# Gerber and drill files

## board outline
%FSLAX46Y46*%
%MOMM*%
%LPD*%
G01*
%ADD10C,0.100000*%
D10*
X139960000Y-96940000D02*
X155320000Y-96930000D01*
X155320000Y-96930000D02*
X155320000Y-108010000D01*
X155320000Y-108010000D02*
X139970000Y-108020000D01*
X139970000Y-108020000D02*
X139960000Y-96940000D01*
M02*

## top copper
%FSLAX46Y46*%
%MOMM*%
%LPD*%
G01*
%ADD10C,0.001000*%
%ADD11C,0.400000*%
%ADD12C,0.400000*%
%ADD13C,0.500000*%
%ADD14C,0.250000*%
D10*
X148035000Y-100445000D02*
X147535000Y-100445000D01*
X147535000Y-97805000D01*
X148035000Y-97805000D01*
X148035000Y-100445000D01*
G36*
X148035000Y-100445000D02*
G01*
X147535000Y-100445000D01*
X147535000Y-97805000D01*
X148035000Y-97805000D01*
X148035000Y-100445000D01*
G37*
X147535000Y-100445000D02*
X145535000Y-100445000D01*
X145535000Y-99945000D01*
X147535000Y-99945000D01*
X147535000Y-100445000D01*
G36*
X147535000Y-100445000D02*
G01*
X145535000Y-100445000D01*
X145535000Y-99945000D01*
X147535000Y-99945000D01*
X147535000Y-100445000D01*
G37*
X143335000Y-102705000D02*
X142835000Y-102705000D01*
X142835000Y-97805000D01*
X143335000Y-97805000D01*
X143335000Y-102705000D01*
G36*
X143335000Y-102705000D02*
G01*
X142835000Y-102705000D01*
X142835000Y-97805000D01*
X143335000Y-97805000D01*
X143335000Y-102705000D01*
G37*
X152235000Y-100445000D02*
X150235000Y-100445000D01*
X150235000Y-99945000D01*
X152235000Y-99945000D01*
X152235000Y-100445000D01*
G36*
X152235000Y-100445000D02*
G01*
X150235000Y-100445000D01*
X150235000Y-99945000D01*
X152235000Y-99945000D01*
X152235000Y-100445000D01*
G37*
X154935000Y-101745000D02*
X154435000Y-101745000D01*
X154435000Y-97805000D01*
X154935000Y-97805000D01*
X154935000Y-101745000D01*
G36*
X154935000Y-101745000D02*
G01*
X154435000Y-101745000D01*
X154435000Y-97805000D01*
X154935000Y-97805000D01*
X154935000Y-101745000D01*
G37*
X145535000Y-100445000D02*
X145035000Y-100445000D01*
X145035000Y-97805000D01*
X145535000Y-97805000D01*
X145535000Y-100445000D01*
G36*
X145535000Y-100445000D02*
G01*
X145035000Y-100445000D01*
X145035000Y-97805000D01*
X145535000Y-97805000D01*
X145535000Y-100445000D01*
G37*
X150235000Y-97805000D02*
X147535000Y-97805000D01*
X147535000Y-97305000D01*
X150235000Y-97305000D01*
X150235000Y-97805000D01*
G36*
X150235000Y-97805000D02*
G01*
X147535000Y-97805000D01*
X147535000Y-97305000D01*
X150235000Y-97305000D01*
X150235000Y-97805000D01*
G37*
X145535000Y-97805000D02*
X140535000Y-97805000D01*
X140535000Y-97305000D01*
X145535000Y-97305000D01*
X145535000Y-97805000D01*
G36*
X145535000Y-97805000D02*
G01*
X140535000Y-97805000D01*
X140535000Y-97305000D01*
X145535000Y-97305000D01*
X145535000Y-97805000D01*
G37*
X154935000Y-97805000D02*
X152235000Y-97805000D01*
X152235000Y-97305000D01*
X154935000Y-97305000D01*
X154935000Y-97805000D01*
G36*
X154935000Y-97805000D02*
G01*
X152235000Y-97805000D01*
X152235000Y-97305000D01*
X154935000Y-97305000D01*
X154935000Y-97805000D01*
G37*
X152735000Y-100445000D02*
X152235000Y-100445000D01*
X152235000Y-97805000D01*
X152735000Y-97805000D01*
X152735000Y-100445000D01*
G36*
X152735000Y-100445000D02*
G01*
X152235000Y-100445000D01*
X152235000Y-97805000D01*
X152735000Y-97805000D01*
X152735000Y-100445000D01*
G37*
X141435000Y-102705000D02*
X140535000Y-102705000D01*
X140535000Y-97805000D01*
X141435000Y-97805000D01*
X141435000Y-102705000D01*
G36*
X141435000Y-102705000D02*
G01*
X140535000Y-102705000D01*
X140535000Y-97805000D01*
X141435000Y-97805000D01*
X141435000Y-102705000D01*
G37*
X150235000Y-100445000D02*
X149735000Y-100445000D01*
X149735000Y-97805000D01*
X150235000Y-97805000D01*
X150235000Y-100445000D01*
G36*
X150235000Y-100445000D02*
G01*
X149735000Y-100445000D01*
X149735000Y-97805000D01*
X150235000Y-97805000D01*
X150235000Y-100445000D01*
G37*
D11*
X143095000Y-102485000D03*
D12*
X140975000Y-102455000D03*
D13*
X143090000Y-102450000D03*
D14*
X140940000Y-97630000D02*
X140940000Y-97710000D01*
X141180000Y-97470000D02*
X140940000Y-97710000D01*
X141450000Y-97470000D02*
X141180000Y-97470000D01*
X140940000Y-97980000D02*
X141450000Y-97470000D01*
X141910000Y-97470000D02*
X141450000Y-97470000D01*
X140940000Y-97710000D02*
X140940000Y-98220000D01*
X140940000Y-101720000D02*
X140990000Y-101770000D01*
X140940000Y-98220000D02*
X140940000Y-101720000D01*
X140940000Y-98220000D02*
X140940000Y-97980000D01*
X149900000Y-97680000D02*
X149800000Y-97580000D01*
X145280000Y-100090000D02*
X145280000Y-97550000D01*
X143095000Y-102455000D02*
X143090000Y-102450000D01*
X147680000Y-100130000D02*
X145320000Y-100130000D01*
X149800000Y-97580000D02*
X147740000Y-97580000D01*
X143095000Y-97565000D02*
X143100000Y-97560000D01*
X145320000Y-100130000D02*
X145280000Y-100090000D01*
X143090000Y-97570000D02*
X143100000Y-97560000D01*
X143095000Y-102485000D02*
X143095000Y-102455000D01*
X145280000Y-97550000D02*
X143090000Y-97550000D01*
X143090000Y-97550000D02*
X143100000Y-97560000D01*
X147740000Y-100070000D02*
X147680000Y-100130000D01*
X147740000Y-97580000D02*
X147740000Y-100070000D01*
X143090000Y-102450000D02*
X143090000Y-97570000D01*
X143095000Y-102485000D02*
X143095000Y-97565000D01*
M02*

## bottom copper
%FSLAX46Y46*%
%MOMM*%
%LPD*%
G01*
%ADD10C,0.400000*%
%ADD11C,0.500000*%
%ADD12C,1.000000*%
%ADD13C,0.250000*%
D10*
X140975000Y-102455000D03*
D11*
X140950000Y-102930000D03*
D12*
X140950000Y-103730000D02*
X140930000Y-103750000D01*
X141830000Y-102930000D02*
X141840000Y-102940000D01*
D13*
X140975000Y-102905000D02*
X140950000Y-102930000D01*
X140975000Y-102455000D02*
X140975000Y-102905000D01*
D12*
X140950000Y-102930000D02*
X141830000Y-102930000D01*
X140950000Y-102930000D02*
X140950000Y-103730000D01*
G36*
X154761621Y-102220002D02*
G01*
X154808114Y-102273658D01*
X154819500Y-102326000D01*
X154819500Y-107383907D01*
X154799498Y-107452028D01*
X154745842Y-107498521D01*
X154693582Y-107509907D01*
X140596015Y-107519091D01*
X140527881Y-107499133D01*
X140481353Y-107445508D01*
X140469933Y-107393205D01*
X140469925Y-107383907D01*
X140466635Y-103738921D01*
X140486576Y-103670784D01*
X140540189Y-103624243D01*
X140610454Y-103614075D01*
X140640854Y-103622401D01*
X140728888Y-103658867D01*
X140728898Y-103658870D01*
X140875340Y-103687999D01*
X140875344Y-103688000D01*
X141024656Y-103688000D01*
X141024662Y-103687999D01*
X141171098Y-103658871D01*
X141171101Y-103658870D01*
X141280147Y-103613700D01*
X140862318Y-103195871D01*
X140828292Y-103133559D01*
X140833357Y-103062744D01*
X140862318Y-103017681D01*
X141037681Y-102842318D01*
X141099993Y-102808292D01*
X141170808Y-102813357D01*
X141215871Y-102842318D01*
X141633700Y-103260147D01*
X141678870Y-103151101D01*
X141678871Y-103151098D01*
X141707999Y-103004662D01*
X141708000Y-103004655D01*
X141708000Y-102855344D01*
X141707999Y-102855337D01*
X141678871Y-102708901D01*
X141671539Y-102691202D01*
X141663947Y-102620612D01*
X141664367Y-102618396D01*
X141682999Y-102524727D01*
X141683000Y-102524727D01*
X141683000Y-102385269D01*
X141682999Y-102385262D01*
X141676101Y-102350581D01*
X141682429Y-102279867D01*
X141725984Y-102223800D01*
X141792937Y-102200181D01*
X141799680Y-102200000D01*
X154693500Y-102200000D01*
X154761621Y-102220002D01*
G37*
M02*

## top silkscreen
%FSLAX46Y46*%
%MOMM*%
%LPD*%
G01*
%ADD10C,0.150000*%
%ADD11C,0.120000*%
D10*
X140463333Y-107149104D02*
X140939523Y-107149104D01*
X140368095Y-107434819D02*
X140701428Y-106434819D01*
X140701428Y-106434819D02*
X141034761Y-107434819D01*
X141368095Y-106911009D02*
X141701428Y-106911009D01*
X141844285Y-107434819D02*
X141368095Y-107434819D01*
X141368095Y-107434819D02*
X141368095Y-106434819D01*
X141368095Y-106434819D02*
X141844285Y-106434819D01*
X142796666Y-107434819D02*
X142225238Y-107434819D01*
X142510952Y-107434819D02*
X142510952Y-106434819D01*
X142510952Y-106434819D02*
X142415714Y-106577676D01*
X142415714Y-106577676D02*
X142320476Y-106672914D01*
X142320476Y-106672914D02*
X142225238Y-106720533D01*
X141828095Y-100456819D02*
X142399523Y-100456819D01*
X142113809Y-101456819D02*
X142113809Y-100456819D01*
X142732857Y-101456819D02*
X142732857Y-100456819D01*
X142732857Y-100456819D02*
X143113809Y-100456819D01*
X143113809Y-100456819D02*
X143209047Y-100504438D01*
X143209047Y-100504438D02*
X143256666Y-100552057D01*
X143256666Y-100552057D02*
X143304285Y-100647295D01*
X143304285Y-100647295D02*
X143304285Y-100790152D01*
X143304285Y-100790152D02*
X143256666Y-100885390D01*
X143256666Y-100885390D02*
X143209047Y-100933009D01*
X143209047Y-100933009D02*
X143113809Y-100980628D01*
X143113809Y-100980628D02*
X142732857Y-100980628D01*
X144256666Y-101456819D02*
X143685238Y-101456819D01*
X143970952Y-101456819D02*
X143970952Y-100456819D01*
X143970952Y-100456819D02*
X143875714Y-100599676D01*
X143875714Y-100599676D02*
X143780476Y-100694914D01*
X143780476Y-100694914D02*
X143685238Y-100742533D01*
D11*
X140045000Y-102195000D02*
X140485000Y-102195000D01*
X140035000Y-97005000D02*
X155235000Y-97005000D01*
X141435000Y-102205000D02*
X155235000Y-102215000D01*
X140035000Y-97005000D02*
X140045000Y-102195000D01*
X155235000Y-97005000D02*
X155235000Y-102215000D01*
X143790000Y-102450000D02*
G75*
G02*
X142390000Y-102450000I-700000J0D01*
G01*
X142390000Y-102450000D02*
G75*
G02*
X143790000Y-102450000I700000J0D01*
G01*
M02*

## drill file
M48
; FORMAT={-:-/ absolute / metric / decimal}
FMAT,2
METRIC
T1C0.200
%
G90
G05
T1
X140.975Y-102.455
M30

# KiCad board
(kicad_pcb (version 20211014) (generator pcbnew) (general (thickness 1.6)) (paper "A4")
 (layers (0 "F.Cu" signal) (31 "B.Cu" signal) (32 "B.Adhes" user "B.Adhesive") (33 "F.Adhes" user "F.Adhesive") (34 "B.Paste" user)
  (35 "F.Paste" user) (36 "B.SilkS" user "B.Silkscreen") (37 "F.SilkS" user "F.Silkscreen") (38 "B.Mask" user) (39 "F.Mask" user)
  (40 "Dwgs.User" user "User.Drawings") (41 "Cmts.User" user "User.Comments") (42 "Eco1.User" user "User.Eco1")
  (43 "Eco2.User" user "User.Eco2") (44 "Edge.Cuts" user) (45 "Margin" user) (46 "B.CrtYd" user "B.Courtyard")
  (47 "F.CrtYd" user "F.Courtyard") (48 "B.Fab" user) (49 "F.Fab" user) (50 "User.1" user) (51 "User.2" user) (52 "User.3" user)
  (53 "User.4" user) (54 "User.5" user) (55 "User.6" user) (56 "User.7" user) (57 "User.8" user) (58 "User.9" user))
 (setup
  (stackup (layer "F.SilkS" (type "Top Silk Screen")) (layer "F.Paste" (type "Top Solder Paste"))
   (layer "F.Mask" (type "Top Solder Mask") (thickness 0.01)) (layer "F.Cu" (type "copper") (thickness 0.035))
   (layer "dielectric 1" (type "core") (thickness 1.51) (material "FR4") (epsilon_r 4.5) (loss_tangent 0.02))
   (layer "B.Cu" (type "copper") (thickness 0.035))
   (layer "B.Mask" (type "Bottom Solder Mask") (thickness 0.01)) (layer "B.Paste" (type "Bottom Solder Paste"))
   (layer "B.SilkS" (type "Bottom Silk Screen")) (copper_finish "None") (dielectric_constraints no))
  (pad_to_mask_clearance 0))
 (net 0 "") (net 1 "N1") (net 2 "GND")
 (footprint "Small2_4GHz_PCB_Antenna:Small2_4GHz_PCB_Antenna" (layer "F.Cu") (at 140.535 97.305)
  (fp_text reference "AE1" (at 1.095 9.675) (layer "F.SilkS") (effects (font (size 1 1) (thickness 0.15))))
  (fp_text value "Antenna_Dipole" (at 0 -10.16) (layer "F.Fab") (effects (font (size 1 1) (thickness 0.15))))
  (fp_poly (pts (xy 7.5 3.14) (xy 7 3.14) (xy 7 0.5) (xy 7.5 0.5)) (layer "F.Cu") (width 0.001) (fill solid))
  (fp_poly (pts (xy 7 3.14) (xy 5 3.14) (xy 5 2.64) (xy 7 2.64)) (layer "F.Cu") (width 0.001) (fill solid))
  (fp_poly (pts (xy 2.8 5.4) (xy 2.3 5.4) (xy 2.3 0.5) (xy 2.8 0.5)) (layer "F.Cu") (width 0.001) (fill solid))
  (fp_poly (pts (xy 11.7 3.14) (xy 9.7 3.14) (xy 9.7 2.64) (xy 11.7 2.64)) (layer "F.Cu") (width 0.001) (fill solid))
  (fp_poly (pts (xy 14.4 4.44) (xy 13.9 4.44) (xy 13.9 0.5) (xy 14.4 0.5)) (layer "F.Cu") (width 0.001) (fill solid))
  (fp_poly (pts (xy 5 3.14) (xy 4.5 3.14) (xy 4.5 0.5) (xy 5 0.5)) (layer "F.Cu") (width 0.001) (fill solid))
  (fp_poly (pts (xy 9.7 0.5) (xy 7 0.5) (xy 7 0) (xy 9.7 0)) (layer "F.Cu") (width 0.001) (fill solid))
  (fp_poly (pts (xy 5 0.5) (xy 0 0.5) (xy 0 0) (xy 5 0)) (layer "F.Cu") (width 0.001) (fill solid))
  (fp_poly (pts (xy 14.4 0.5) (xy 11.7 0.5) (xy 11.7 0) (xy 14.4 0)) (layer "F.Cu") (width 0.001) (fill solid))
  (fp_poly (pts (xy 12.2 3.14) (xy 11.7 3.14) (xy 11.7 0.5) (xy 12.2 0.5)) (layer "F.Cu") (width 0.001) (fill solid))
  (fp_poly (pts (xy 0.9 5.4) (xy 0 5.4) (xy 0 0.5) (xy 0.9 0.5)) (layer "F.Cu") (width 0.001) (fill solid))
  (fp_poly (pts (xy 9.7 3.14) (xy 9.2 3.14) (xy 9.2 0.5) (xy 9.7 0.5)) (layer "F.Cu") (width 0.001) (fill solid))
  (fp_line (start -0.49 4.89) (end -0.05 4.89) (layer "F.SilkS") (width 0.12))
  (fp_line (start -0.5 -0.3) (end 14.7 -0.3) (layer "F.SilkS") (width 0.12))
  (fp_line (start 0.9 4.9) (end 14.7 4.91) (layer "F.SilkS") (width 0.12))
  (fp_line (start -0.5 -0.3) (end -0.49 4.89) (layer "F.SilkS") (width 0.12))
  (fp_line (start 14.7 -0.3) (end 14.7 4.91) (layer "F.SilkS") (width 0.12))
  (pad "1" smd circle locked (at 2.56 5.18) (size 0.4 0.4) (layers "F.Cu" "F.Paste" "F.Mask") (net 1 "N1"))
  (pad "2" thru_hole circle locked (at 0.44 5.15) (size 0.4 0.4) (drill 0.2) (layers *.Cu *.Mask) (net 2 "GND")))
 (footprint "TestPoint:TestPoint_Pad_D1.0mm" (layer "F.Cu") (at 143.09 102.45)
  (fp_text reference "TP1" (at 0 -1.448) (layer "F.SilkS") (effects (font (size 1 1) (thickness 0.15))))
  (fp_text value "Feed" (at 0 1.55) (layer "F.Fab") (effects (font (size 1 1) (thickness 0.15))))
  (fp_circle (center 0 0) (end 0 0.7) (layer "F.SilkS") (width 0.12) (fill none))
  (pad "1" smd circle (at 0 0) (size 0.5 0.5) (layers "F.Cu" "F.Mask") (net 1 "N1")))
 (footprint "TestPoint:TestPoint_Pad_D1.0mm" (layer "B.Cu") (at 140.95 102.93 180)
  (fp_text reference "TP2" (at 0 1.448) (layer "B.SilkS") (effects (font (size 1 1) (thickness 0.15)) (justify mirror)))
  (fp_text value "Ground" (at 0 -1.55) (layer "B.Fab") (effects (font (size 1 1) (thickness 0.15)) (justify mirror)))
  (pad "1" smd circle (at 0 0 180) (size 0.5 0.5) (layers "B.Cu" "B.Mask") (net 2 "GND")))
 (gr_line (start 139.96 96.94) (end 155.32 96.93) (layer "Edge.Cuts") (width 0.1))
 (gr_line (start 155.32 96.93) (end 155.32 108.01) (layer "Edge.Cuts") (width 0.1))
 (gr_line (start 155.32 108.01) (end 139.97 108.02) (layer "Edge.Cuts") (width 0.1))
 (gr_line (start 139.97 108.02) (end 139.96 96.94) (layer "Edge.Cuts") (width 0.1))
 (segment (start 140.94 97.63) (end 140.94 97.71) (width 0.25) (layer "F.Cu") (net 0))
 (segment (start 141.18 97.47) (end 140.94 97.71) (width 0.25) (layer "F.Cu") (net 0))
 (segment (start 141.45 97.47) (end 141.18 97.47) (width 0.25) (layer "F.Cu") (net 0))
 (segment (start 140.94 97.98) (end 141.45 97.47) (width 0.25) (layer "F.Cu") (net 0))
 (segment (start 141.91 97.47) (end 141.45 97.47) (width 0.25) (layer "F.Cu") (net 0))
 (segment (start 140.94 97.71) (end 140.94 98.22) (width 0.25) (layer "F.Cu") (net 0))
 (segment (start 140.94 101.72) (end 140.99 101.77) (width 0.25) (layer "F.Cu") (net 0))
 (segment (start 140.94 98.22) (end 140.94 101.72) (width 0.25) (layer "F.Cu") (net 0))
 (segment (start 140.94 98.22) (end 140.94 97.98) (width 0.25) (layer "F.Cu") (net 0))
 (segment (start 140.95 103.73) (end 140.93 103.75) (width 1) (layer "B.Cu") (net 2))
 (segment (start 141.83 102.93) (end 141.84 102.94) (width 1) (layer "B.Cu") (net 2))
 (segment (start 140.975 102.905) (end 140.95 102.93) (width 0.25) (layer "B.Cu") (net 2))
 (segment (start 140.975 102.455) (end 140.975 102.905) (width 0.25) (layer "B.Cu") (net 2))
 (segment (start 140.95 102.93) (end 141.83 102.93) (width 1) (layer "B.Cu") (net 2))
 (segment (start 140.95 102.93) (end 140.95 103.73) (width 1) (layer "B.Cu") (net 2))
 (segment (start 149.9 97.68) (end 149.8 97.58) (width 0.25) (layer "F.Cu") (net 1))
 (segment (start 145.28 100.09) (end 145.28 97.55) (width 0.25) (layer "F.Cu") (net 1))
 (segment (start 143.095 102.455) (end 143.09 102.45) (width 0.25) (layer "F.Cu") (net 1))
 (segment (start 147.68 100.13) (end 145.32 100.13) (width 0.25) (layer "F.Cu") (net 1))
 (segment (start 149.8 97.58) (end 147.74 97.58) (width 0.25) (layer "F.Cu") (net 1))
 (segment (start 143.095 97.565) (end 143.1 97.56) (width 0.25) (layer "F.Cu") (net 1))
 (segment (start 145.32 100.13) (end 145.28 100.09) (width 0.25) (layer "F.Cu") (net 1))
 (segment (start 143.09 97.57) (end 143.1 97.56) (width 0.25) (layer "F.Cu") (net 1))
 (segment (start 143.095 102.485) (end 143.095 102.455) (width 0.25) (layer "F.Cu") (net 1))
 (segment (start 145.28 97.55) (end 143.09 97.55) (width 0.25) (layer "F.Cu") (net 1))
 (segment (start 143.09 97.55) (end 143.1 97.56) (width 0.25) (layer "F.Cu") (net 1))
 (segment (start 147.74 100.07) (end 147.68 100.13) (width 0.25) (layer "F.Cu") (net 1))
 (segment (start 147.74 97.58) (end 147.74 100.07) (width 0.25) (layer "F.Cu") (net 1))
 (segment (start 143.09 102.45) (end 143.09 97.57) (width 0.25) (layer "F.Cu") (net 1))
 (segment (start 143.095 102.485) (end 143.095 97.565) (width 0.25) (layer "F.Cu") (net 1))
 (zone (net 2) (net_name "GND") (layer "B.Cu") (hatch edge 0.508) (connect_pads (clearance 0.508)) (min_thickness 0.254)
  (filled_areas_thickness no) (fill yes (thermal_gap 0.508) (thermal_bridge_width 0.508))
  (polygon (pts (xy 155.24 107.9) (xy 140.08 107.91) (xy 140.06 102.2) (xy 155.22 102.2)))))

